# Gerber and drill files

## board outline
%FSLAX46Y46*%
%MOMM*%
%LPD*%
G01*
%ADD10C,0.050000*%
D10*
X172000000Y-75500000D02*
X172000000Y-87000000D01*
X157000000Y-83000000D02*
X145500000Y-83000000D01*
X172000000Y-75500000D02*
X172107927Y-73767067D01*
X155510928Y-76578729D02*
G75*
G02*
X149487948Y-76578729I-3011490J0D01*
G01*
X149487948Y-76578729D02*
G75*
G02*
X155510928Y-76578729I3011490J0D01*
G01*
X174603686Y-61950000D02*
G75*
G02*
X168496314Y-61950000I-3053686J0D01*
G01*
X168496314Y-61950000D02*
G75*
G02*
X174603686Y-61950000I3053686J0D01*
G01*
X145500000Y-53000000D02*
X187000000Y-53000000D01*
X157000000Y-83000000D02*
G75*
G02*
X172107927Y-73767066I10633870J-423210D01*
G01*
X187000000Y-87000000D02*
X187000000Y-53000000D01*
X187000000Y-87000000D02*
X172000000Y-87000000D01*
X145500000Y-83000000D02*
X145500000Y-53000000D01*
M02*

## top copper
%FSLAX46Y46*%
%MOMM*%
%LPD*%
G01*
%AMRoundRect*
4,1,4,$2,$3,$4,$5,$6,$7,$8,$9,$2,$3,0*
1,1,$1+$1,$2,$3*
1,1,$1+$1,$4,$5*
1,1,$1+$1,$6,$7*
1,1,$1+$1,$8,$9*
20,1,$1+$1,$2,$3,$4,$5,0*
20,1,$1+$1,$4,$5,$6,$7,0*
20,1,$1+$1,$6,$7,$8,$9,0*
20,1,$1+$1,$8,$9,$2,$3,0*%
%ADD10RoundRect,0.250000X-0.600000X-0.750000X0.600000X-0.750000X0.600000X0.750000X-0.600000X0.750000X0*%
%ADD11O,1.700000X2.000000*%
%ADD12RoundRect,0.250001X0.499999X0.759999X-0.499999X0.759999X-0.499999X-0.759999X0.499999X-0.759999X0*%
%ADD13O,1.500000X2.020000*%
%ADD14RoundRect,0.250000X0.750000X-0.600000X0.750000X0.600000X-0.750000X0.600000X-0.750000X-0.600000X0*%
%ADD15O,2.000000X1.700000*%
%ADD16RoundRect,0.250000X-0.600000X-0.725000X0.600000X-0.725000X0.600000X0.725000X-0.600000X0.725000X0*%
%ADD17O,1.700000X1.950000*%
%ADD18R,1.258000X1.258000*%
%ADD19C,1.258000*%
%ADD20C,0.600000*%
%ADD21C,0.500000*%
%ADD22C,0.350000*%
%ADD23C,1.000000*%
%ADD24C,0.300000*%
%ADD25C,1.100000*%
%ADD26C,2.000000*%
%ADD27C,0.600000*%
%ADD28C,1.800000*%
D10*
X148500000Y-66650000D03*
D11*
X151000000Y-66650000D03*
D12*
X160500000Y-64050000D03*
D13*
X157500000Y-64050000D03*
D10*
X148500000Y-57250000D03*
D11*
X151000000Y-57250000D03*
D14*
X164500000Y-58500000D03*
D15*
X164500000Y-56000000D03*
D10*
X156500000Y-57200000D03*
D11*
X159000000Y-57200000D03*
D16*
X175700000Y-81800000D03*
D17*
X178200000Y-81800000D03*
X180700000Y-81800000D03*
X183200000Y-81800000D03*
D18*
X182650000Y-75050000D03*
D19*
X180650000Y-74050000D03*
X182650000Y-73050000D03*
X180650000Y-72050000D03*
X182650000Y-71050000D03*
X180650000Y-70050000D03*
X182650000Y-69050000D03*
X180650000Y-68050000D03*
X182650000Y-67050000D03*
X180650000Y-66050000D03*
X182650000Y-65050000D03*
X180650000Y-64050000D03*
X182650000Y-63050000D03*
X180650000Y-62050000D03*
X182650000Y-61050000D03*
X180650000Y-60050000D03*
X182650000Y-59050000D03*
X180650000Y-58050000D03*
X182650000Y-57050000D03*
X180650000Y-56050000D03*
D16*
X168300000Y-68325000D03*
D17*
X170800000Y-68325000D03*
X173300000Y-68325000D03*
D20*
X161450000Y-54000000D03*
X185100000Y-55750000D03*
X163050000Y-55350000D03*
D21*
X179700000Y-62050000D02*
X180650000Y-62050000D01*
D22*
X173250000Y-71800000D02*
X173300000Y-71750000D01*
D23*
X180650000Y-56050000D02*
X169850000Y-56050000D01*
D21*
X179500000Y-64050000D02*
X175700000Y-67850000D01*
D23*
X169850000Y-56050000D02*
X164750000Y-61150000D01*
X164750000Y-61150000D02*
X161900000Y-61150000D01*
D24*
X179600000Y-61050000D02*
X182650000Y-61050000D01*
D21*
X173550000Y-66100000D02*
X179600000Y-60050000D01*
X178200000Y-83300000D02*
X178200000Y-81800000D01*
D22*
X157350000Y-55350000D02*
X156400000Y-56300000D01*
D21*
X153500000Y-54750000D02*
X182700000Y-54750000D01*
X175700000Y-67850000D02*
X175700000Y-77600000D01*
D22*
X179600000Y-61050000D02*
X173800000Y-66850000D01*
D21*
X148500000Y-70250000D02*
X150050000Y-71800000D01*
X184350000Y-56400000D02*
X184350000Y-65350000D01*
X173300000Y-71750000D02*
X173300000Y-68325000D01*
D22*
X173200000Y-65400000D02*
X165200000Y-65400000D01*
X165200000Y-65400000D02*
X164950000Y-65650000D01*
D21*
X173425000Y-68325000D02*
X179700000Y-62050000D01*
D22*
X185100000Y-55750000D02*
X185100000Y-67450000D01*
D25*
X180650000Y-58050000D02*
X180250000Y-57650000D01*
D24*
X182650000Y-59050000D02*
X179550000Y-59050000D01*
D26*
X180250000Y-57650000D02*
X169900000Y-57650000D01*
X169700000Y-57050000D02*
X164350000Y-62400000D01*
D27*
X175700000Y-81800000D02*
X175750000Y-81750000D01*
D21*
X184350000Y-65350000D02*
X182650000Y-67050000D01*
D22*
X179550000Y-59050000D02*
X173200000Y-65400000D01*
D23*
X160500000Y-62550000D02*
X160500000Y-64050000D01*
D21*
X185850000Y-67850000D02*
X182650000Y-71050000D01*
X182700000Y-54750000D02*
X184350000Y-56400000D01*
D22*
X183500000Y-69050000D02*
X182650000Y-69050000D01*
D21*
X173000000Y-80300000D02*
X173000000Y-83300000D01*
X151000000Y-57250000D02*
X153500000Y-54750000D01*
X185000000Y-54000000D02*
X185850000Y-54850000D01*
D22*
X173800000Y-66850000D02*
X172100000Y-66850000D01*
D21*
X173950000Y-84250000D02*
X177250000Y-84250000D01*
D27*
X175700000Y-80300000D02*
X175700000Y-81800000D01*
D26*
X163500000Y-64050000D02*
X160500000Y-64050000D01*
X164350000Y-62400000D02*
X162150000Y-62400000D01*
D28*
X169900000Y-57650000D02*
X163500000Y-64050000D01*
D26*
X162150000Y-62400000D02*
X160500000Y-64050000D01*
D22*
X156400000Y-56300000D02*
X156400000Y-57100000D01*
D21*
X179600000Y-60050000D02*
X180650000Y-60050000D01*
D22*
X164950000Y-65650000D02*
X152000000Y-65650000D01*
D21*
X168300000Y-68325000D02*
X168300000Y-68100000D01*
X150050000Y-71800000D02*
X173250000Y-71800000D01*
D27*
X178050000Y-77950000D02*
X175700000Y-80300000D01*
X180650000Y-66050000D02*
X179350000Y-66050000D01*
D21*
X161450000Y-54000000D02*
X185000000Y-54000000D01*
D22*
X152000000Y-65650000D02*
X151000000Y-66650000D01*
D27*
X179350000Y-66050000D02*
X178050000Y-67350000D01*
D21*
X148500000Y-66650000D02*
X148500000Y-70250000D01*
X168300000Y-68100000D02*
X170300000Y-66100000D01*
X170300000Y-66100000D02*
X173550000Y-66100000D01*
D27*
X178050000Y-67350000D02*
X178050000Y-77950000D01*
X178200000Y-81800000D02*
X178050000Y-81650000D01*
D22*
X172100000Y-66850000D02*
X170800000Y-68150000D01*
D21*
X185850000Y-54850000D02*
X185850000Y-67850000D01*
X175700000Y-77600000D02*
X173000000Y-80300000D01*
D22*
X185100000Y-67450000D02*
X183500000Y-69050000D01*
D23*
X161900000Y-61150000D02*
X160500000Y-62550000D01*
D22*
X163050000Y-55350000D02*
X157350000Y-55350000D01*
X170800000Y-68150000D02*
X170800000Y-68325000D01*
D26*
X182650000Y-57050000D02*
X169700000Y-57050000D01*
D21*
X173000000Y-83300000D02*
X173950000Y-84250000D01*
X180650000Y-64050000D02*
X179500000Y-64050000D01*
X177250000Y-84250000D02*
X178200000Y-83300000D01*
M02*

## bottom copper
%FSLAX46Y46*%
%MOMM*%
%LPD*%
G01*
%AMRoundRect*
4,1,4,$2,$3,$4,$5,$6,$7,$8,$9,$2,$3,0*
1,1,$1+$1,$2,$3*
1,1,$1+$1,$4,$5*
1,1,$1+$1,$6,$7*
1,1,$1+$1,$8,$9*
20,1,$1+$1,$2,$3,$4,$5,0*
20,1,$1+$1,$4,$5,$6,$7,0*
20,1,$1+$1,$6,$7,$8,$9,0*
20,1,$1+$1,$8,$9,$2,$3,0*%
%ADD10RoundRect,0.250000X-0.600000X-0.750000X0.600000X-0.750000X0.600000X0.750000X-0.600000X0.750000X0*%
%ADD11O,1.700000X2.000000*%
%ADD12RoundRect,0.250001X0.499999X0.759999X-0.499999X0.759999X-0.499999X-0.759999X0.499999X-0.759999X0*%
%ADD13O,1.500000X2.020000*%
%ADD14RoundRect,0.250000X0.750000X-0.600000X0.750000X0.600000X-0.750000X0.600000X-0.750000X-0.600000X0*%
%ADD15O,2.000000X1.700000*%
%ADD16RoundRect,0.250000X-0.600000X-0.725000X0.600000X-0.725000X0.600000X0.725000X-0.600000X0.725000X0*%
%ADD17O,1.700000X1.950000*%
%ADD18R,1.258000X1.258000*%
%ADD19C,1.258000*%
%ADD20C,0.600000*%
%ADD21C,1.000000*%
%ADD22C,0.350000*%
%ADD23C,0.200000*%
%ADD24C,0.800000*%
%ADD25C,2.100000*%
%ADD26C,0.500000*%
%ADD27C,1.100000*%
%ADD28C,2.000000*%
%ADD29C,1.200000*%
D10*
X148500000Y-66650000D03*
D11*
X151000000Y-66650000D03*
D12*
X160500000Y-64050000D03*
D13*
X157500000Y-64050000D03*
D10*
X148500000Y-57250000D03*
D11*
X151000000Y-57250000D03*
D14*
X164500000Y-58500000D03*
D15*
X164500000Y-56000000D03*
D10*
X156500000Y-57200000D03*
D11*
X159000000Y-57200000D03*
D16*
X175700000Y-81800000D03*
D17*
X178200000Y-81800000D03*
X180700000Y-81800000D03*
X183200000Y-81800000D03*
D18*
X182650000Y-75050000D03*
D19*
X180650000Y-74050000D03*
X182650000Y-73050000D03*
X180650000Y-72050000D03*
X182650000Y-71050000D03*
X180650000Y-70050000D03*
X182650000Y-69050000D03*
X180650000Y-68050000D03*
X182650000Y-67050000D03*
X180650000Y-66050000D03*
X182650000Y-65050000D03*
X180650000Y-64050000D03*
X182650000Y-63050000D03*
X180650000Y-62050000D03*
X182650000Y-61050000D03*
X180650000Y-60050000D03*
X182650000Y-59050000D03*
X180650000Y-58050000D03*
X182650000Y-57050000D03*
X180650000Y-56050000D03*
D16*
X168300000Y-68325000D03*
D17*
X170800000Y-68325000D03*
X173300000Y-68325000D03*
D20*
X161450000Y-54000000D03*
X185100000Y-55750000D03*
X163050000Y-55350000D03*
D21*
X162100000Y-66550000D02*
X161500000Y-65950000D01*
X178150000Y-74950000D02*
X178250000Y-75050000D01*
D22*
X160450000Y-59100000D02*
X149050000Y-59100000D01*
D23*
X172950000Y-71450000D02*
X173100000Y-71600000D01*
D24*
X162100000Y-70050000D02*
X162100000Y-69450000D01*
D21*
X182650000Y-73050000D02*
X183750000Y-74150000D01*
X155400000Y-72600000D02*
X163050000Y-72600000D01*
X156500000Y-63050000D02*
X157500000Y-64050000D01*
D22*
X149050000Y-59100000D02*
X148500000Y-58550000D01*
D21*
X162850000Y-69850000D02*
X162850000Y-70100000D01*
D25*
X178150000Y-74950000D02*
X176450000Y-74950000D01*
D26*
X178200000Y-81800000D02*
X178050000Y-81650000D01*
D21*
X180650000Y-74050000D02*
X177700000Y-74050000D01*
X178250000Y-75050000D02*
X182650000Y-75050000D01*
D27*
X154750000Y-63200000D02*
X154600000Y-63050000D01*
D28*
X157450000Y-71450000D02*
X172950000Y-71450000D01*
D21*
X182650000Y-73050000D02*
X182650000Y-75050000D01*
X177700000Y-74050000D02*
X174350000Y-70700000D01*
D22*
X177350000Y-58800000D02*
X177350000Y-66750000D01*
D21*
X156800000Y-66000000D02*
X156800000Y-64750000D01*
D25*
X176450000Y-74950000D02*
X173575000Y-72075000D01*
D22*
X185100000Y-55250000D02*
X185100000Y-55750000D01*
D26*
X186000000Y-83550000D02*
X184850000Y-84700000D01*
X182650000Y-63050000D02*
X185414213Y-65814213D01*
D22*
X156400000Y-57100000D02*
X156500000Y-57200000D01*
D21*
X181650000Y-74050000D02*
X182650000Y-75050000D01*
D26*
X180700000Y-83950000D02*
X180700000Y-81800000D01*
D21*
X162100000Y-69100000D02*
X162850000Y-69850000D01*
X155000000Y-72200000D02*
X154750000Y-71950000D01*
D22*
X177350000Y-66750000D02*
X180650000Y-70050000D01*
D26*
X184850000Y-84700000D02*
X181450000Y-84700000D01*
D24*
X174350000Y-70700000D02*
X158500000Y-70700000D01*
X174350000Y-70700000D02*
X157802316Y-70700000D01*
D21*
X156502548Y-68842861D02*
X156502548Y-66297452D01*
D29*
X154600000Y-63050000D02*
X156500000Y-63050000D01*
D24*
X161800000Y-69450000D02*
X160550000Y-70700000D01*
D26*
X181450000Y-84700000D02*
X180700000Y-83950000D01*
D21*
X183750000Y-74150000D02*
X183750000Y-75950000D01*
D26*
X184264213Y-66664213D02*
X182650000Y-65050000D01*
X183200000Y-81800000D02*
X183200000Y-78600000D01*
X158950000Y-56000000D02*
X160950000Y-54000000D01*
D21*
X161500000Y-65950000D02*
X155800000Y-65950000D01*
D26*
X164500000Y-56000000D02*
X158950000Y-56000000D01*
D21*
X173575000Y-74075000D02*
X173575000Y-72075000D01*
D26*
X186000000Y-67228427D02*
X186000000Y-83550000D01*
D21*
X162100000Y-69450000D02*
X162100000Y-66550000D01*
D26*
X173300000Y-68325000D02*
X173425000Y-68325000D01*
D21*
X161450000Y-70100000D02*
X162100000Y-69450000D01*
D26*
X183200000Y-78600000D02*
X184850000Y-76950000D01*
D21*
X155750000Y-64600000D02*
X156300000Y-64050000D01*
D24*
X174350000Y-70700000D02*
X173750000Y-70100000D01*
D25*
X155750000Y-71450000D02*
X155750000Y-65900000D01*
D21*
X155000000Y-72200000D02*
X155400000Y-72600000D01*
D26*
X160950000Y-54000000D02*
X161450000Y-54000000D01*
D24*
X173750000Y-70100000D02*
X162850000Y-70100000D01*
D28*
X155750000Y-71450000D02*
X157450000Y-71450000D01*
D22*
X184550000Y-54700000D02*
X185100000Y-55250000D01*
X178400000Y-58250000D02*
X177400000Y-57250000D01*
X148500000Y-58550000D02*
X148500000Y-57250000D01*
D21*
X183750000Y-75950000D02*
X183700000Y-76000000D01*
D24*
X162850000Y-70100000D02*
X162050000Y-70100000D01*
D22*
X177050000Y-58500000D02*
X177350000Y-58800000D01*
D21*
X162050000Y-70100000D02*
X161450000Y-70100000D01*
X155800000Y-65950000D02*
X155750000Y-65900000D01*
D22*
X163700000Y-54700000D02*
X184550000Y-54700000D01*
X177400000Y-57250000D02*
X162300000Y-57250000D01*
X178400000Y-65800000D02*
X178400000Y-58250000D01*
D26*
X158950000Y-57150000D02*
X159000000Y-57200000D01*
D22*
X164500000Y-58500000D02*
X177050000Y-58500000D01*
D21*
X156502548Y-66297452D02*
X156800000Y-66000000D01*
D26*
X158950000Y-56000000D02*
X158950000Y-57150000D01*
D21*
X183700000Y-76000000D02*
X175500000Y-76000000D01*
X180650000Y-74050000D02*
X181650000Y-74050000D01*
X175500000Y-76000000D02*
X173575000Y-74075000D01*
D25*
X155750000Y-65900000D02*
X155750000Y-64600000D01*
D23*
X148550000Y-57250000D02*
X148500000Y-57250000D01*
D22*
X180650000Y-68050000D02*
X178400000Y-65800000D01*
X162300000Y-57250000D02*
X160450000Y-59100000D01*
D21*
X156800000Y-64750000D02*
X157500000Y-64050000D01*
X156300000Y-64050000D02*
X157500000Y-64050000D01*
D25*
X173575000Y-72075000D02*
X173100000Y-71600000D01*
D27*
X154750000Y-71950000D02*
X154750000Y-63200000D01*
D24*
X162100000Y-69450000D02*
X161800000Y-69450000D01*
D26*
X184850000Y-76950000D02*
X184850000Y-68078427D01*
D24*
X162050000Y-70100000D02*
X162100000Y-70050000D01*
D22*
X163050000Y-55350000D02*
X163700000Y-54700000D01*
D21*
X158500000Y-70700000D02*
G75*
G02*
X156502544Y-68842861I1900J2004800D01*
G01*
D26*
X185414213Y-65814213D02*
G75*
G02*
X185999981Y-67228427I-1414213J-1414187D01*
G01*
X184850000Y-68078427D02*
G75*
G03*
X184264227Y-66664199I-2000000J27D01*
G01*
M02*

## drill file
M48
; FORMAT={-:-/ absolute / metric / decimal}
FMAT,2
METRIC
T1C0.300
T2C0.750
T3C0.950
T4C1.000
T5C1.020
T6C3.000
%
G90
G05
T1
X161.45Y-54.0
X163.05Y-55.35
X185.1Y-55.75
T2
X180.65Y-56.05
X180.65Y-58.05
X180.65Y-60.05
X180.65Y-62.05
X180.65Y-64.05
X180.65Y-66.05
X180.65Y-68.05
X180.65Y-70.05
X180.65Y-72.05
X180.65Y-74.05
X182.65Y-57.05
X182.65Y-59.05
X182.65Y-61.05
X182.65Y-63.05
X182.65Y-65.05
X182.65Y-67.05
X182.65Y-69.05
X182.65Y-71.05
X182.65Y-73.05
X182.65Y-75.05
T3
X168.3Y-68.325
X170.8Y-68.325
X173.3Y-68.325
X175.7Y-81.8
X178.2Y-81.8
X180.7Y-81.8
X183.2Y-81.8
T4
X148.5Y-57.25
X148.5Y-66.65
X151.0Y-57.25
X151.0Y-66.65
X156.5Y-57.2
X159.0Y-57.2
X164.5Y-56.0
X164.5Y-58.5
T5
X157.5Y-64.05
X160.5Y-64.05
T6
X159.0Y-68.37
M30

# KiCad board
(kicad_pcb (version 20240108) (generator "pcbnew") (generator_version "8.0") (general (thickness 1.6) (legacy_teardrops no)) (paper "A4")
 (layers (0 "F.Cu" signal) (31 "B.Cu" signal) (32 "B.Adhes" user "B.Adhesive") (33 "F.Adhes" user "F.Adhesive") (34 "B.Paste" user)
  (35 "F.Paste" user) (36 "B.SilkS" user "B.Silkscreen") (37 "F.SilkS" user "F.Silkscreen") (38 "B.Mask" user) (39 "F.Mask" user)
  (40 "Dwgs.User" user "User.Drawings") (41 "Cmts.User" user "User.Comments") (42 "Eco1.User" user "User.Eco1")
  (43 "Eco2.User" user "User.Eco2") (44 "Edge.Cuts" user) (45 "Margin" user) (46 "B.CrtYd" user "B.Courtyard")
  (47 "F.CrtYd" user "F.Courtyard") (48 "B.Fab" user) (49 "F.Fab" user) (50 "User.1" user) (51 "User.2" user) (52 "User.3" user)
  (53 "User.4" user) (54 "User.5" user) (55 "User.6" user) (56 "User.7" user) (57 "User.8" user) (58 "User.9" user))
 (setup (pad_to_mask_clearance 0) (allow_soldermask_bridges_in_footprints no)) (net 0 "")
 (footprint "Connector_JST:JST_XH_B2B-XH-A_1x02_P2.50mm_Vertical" (layer "F.Cu") (at 148.5 66.65)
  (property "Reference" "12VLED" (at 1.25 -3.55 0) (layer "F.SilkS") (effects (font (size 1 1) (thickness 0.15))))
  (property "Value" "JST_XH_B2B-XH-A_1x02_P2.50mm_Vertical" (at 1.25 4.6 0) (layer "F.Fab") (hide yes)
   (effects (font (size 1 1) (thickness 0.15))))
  (pad "1" thru_hole roundrect (at 0 0) (size 1.7 2) (drill 1) (layers "*.Cu" "*.Mask") (remove_unused_layers no)
   (roundrect_rratio 0.147059))
  (pad "2" thru_hole oval (at 2.5 0) (size 1.7 2) (drill 1) (layers "*.Cu" "*.Mask") (remove_unused_layers no)))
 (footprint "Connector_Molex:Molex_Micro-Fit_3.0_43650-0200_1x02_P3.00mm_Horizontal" (layer "F.Cu") (at 160.5 64.05 180)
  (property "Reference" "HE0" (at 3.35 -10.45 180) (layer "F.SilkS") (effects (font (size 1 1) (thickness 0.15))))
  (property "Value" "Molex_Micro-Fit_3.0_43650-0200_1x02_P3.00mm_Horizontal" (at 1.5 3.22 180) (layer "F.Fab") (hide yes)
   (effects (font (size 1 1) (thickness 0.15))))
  (pad "" np_thru_hole circle (at 1.5 -4.32 180) (size 3 3) (drill 3) (layers "*.Cu" "*.Mask"))
  (pad "1" thru_hole roundrect (at 0 0 180) (size 1.5 2.02) (drill 1.02) (layers "*.Cu" "*.Mask") (remove_unused_layers no)
   (roundrect_rratio 0.166667))
  (pad "2" thru_hole oval (at 3 0 180) (size 1.5 2.02) (drill 1.02) (layers "*.Cu" "*.Mask") (remove_unused_layers no)))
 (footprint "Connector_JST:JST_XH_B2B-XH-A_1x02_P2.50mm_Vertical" (layer "F.Cu") (at 148.5 57.25)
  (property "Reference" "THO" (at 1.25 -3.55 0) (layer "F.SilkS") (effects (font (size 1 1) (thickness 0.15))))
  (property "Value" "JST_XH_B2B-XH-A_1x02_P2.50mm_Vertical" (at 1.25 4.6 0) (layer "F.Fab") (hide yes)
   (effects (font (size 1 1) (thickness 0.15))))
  (pad "1" thru_hole roundrect (at 0 0) (size 1.7 2) (drill 1) (layers "*.Cu" "*.Mask") (remove_unused_layers no)
   (roundrect_rratio 0.147059))
  (pad "2" thru_hole oval (at 2.5 0) (size 1.7 2) (drill 1) (layers "*.Cu" "*.Mask") (remove_unused_layers no)))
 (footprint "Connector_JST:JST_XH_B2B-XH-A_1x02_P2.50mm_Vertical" (layer "F.Cu") (at 164.5 58.5 90)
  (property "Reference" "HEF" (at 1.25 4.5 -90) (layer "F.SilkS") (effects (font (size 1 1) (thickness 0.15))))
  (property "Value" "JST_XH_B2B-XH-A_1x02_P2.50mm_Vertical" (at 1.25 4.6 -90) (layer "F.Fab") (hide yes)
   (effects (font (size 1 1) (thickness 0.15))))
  (pad "1" thru_hole roundrect (at 0 0 90) (size 1.7 2) (drill 1) (layers "*.Cu" "*.Mask") (remove_unused_layers no)
   (roundrect_rratio 0.147059))
  (pad "2" thru_hole oval (at 2.5 0 90) (size 1.7 2) (drill 1) (layers "*.Cu" "*.Mask") (remove_unused_layers no)))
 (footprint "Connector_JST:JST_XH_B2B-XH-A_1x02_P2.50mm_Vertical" (layer "F.Cu") (at 156.5 57.2)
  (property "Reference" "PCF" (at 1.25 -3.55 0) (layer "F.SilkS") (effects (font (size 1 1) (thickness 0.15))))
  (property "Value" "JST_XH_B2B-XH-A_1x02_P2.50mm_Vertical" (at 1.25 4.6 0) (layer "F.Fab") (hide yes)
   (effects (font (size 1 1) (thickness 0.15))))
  (pad "1" thru_hole roundrect (at 0 0) (size 1.7 2) (drill 1) (layers "*.Cu" "*.Mask") (remove_unused_layers no)
   (roundrect_rratio 0.147059))
  (pad "2" thru_hole oval (at 2.5 0) (size 1.7 2) (drill 1) (layers "*.Cu" "*.Mask") (remove_unused_layers no)))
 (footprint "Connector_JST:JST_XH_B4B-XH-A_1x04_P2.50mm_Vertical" (layer "F.Cu") (at 175.7 81.8)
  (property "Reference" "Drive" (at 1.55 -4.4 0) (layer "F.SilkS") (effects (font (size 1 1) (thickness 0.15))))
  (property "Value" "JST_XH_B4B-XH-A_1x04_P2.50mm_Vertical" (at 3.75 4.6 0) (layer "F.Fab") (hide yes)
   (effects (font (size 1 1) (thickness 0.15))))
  (pad "1" thru_hole roundrect (at 0 0) (size 1.7 1.95) (drill 0.95) (layers "*.Cu" "*.Mask") (remove_unused_layers no)
   (roundrect_rratio 0.147059))
  (pad "2" thru_hole oval (at 2.5 0) (size 1.7 1.95) (drill 0.95) (layers "*.Cu" "*.Mask") (remove_unused_layers no))
  (pad "3" thru_hole oval (at 5 0) (size 1.7 1.95) (drill 0.95) (layers "*.Cu" "*.Mask") (remove_unused_layers no))
  (pad "4" thru_hole oval (at 7.5 0) (size 1.7 1.95) (drill 0.95) (layers "*.Cu" "*.Mask") (remove_unused_layers no)))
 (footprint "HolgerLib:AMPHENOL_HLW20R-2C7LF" (layer "F.Cu") (at 183.225 65.55 90)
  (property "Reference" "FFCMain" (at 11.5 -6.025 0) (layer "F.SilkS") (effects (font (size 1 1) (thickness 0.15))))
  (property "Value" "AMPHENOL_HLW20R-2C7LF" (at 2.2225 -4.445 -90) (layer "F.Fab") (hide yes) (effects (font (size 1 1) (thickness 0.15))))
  (pad "1" thru_hole rect (at -9.5 -0.575 90) (size 1.258 1.258) (drill 0.75) (layers "*.Cu" "*.Mask") (remove_unused_layers no)
   (solder_mask_margin 0.102))
  (pad "2" thru_hole circle (at -8.5 -2.575 90) (size 1.258 1.258) (drill 0.75) (layers "*.Cu" "*.Mask") (remove_unused_layers no)
   (solder_mask_margin 0.102))
  (pad "3" thru_hole circle (at -7.5 -0.575 90) (size 1.258 1.258) (drill 0.75) (layers "*.Cu" "*.Mask") (remove_unused_layers no)
   (solder_mask_margin 0.102))
  (pad "4" thru_hole circle (at -6.5 -2.575 90) (size 1.258 1.258) (drill 0.75) (layers "*.Cu" "*.Mask") (remove_unused_layers no)
   (solder_mask_margin 0.102))
  (pad "5" thru_hole circle (at -5.5 -0.575 90) (size 1.258 1.258) (drill 0.75) (layers "*.Cu" "*.Mask") (remove_unused_layers no)
   (solder_mask_margin 0.102))
  (pad "6" thru_hole circle (at -4.5 -2.575 90) (size 1.258 1.258) (drill 0.75) (layers "*.Cu" "*.Mask") (remove_unused_layers no)
   (solder_mask_margin 0.102))
  (pad "7" thru_hole circle (at -3.5 -0.575 90) (size 1.258 1.258) (drill 0.75) (layers "*.Cu" "*.Mask") (remove_unused_layers no)
   (solder_mask_margin 0.102))
  (pad "8" thru_hole circle (at -2.5 -2.575 90) (size 1.258 1.258) (drill 0.75) (layers "*.Cu" "*.Mask") (remove_unused_layers no)
   (solder_mask_margin 0.102))
  (pad "9" thru_hole circle (at -1.5 -0.575 90) (size 1.258 1.258) (drill 0.75) (layers "*.Cu" "*.Mask") (remove_unused_layers no)
   (solder_mask_margin 0.102))
  (pad "10" thru_hole circle (at -0.5 -2.575 90) (size 1.258 1.258) (drill 0.75) (layers "*.Cu" "*.Mask") (remove_unused_layers no)
   (solder_mask_margin 0.102))
  (pad "11" thru_hole circle (at 0.5 -0.575 90) (size 1.258 1.258) (drill 0.75) (layers "*.Cu" "*.Mask") (remove_unused_layers no)
   (solder_mask_margin 0.102))
  (pad "12" thru_hole circle (at 1.5 -2.575 90) (size 1.258 1.258) (drill 0.75) (layers "*.Cu" "*.Mask") (remove_unused_layers no)
   (solder_mask_margin 0.102))
  (pad "13" thru_hole circle (at 2.5 -0.575 90) (size 1.258 1.258) (drill 0.75) (layers "*.Cu" "*.Mask") (remove_unused_layers no)
   (solder_mask_margin 0.102))
  (pad "14" thru_hole circle (at 3.5 -2.575 90) (size 1.258 1.258) (drill 0.75) (layers "*.Cu" "*.Mask") (remove_unused_layers no)
   (solder_mask_margin 0.102))
  (pad "15" thru_hole circle (at 4.5 -0.575 90) (size 1.258 1.258) (drill 0.75) (layers "*.Cu" "*.Mask") (remove_unused_layers no)
   (solder_mask_margin 0.102))
  (pad "16" thru_hole circle (at 5.5 -2.575 90) (size 1.258 1.258) (drill 0.75) (layers "*.Cu" "*.Mask") (remove_unused_layers no)
   (solder_mask_margin 0.102))
  (pad "17" thru_hole circle (at 6.5 -0.575 90) (size 1.258 1.258) (drill 0.75) (layers "*.Cu" "*.Mask") (remove_unused_layers no)
   (solder_mask_margin 0.102))
  (pad "18" thru_hole circle (at 7.5 -2.575 90) (size 1.258 1.258) (drill 0.75) (layers "*.Cu" "*.Mask") (remove_unused_layers no)
   (solder_mask_margin 0.102))
  (pad "19" thru_hole circle (at 8.5 -0.575 90) (size 1.258 1.258) (drill 0.75) (layers "*.Cu" "*.Mask") (remove_unused_layers no)
   (solder_mask_margin 0.102))
  (pad "20" thru_hole circle (at 9.5 -2.575 90) (size 1.258 1.258) (drill 0.75) (layers "*.Cu" "*.Mask") (remove_unused_layers no)
   (solder_mask_margin 0.102)))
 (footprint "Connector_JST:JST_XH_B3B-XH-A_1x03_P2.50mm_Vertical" (layer "F.Cu") (at 168.3 68.325)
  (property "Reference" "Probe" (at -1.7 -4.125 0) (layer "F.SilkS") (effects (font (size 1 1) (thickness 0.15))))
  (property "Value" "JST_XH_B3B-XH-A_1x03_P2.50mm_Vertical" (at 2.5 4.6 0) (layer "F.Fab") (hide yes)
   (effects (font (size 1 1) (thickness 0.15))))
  (pad "1" thru_hole roundrect (at 0 0) (size 1.7 1.95) (drill 0.95) (layers "*.Cu" "*.Mask") (remove_unused_layers no)
   (roundrect_rratio 0.147059))
  (pad "2" thru_hole oval (at 2.5 0) (size 1.7 1.95) (drill 0.95) (layers "*.Cu" "*.Mask") (remove_unused_layers no))
  (pad "3" thru_hole oval (at 5 0) (size 1.7 1.95) (drill 0.95) (layers "*.Cu" "*.Mask") (remove_unused_layers no)))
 (gr_line (start 172 75.5) (end 172 87) (stroke (width 0.05) (type default)) (layer "Edge.Cuts"))
 (gr_line (start 157 83) (end 145.5 83) (stroke (width 0.05) (type default)) (layer "Edge.Cuts"))
 (gr_line (start 172 75.5) (end 172.107927 73.767067) (stroke (width 0.05) (type default)) (layer "Edge.Cuts"))
 (gr_circle (center 152.499438 76.578729) (end 155.510928 76.578729) (stroke (width 0.05) (type default)) (fill none) (layer "Edge.Cuts"))
 (gr_circle (center 171.55 61.95) (end 173.9 63.9) (stroke (width 0.05) (type default)) (fill none) (layer "Edge.Cuts"))
 (gr_line (start 145.5 53) (end 187 53) (stroke (width 0.05) (type default)) (layer "Edge.Cuts"))
 (gr_arc (start 157 83) (mid 162.084312 74.342422) (end 172.107927 73.767067) (stroke (width 0.05) (type default)) (layer "Edge.Cuts"))
 (gr_line (start 187 87) (end 187 53) (stroke (width 0.05) (type default)) (layer "Edge.Cuts"))
 (gr_line (start 187 87) (end 172 87) (stroke (width 0.05) (type default)) (layer "Edge.Cuts"))
 (gr_line (start 145.5 83) (end 145.5 53) (stroke (width 0.05) (type default)) (layer "Edge.Cuts"))
 (segment (start 179.7 62.05) (end 180.65 62.05) (width 0.5) (layer "F.Cu") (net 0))
 (segment (start 173.25 71.8) (end 173.3 71.75) (width 0.35) (layer "F.Cu") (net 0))
 (segment (start 180.65 56.05) (end 169.85 56.05) (width 1) (layer "F.Cu") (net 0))
 (segment (start 179.5 64.05) (end 175.7 67.85) (width 0.5) (layer "F.Cu") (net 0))
 (segment (start 169.85 56.05) (end 164.75 61.15) (width 1) (layer "F.Cu") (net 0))
 (segment (start 164.75 61.15) (end 161.9 61.15) (width 1) (layer "F.Cu") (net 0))
 (segment (start 179.6 61.05) (end 182.65 61.05) (width 0.3) (layer "F.Cu") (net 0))
 (segment (start 173.55 66.1) (end 179.6 60.05) (width 0.5) (layer "F.Cu") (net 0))
 (segment (start 178.2 83.3) (end 178.2 81.8) (width 0.5) (layer "F.Cu") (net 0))
 (segment (start 157.35 55.35) (end 156.4 56.3) (width 0.35) (layer "F.Cu") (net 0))
 (segment (start 153.5 54.75) (end 182.7 54.75) (width 0.5) (layer "F.Cu") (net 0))
 (segment (start 175.7 67.85) (end 175.7 77.6) (width 0.5) (layer "F.Cu") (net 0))
 (segment (start 179.6 61.05) (end 173.8 66.85) (width 0.35) (layer "F.Cu") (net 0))
 (segment (start 148.5 70.25) (end 150.05 71.8) (width 0.5) (layer "F.Cu") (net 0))
 (segment (start 184.35 56.4) (end 184.35 65.35) (width 0.5) (layer "F.Cu") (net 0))
 (segment (start 173.3 71.75) (end 173.3 68.325) (width 0.5) (layer "F.Cu") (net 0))
 (segment (start 173.2 65.4) (end 165.2 65.4) (width 0.35) (layer "F.Cu") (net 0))
 (segment (start 165.2 65.4) (end 164.95 65.65) (width 0.35) (layer "F.Cu") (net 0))
 (segment (start 173.425 68.325) (end 179.7 62.05) (width 0.5) (layer "F.Cu") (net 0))
 (segment (start 185.1 55.75) (end 185.1 67.45) (width 0.35) (layer "F.Cu") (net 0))
 (segment (start 180.65 58.05) (end 180.25 57.65) (width 1.1) (layer "F.Cu") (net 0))
 (segment (start 182.65 59.05) (end 179.55 59.05) (width 0.3) (layer "F.Cu") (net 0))
 (segment (start 180.25 57.65) (end 169.9 57.65) (width 2) (layer "F.Cu") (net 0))
 (segment (start 169.7 57.05) (end 164.35 62.4) (width 2) (layer "F.Cu") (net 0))
 (segment (start 175.7 81.8) (end 175.75 81.75) (width 0.6) (layer "F.Cu") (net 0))
 (segment (start 184.35 65.35) (end 182.65 67.05) (width 0.5) (layer "F.Cu") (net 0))
 (segment (start 179.55 59.05) (end 173.2 65.4) (width 0.35) (layer "F.Cu") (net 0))
 (segment (start 160.5 62.55) (end 160.5 64.05) (width 1) (layer "F.Cu") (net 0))
 (segment (start 185.85 67.85) (end 182.65 71.05) (width 0.5) (layer "F.Cu") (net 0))
 (segment (start 182.7 54.75) (end 184.35 56.4) (width 0.5) (layer "F.Cu") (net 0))
 (segment (start 183.5 69.05) (end 182.65 69.05) (width 0.35) (layer "F.Cu") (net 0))
 (segment (start 173 80.3) (end 173 83.3) (width 0.5) (layer "F.Cu") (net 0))
 (segment (start 151 57.25) (end 153.5 54.75) (width 0.5) (layer "F.Cu") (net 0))
 (segment (start 185 54) (end 185.85 54.85) (width 0.5) (layer "F.Cu") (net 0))
 (segment (start 173.8 66.85) (end 172.1 66.85) (width 0.35) (layer "F.Cu") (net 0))
 (segment (start 173.95 84.25) (end 177.25 84.25) (width 0.5) (layer "F.Cu") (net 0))
 (segment (start 175.7 80.3) (end 175.7 81.8) (width 0.6) (layer "F.Cu") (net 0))
 (segment (start 163.5 64.05) (end 160.5 64.05) (width 2) (layer "F.Cu") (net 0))
 (segment (start 164.35 62.4) (end 162.15 62.4) (width 2) (layer "F.Cu") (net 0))
 (segment (start 169.9 57.65) (end 163.5 64.05) (width 1.8) (layer "F.Cu") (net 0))
 (segment (start 162.15 62.4) (end 160.5 64.05) (width 2) (layer "F.Cu") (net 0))
 (segment (start 156.4 56.3) (end 156.4 57.1) (width 0.35) (layer "F.Cu") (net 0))
 (segment (start 179.6 60.05) (end 180.65 60.05) (width 0.5) (layer "F.Cu") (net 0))
 (segment (start 164.95 65.65) (end 152 65.65) (width 0.35) (layer "F.Cu") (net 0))
 (segment (start 168.3 68.325) (end 168.3 68.1) (width 0.5) (layer "F.Cu") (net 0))
 (segment (start 150.05 71.8) (end 173.25 71.8) (width 0.5) (layer "F.Cu") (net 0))
 (segment (start 178.05 77.95) (end 175.7 80.3) (width 0.6) (layer "F.Cu") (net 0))
 (segment (start 180.65 66.05) (end 179.35 66.05) (width 0.6) (layer "F.Cu") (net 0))
 (segment (start 161.45 54) (end 185 54) (width 0.5) (layer "F.Cu") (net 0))
 (segment (start 152 65.65) (end 151 66.65) (width 0.35) (layer "F.Cu") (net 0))
 (segment (start 179.35 66.05) (end 178.05 67.35) (width 0.6) (layer "F.Cu") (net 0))
 (segment (start 148.5 66.65) (end 148.5 70.25) (width 0.5) (layer "F.Cu") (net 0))
 (segment (start 168.3 68.1) (end 170.3 66.1) (width 0.5) (layer "F.Cu") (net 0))
 (segment (start 170.3 66.1) (end 173.55 66.1) (width 0.5) (layer "F.Cu") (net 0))
 (segment (start 178.05 67.35) (end 178.05 77.95) (width 0.6) (layer "F.Cu") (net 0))
 (segment (start 178.2 81.8) (end 178.05 81.65) (width 0.6) (layer "F.Cu") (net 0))
 (segment (start 172.1 66.85) (end 170.8 68.15) (width 0.35) (layer "F.Cu") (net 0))
 (segment (start 185.85 54.85) (end 185.85 67.85) (width 0.5) (layer "F.Cu") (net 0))
 (segment (start 175.7 77.6) (end 173 80.3) (width 0.5) (layer "F.Cu") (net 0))
 (segment (start 185.1 67.45) (end 183.5 69.05) (width 0.35) (layer "F.Cu") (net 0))
 (segment (start 161.9 61.15) (end 160.5 62.55) (width 1) (layer "F.Cu") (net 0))
 (segment (start 163.05 55.35) (end 157.35 55.35) (width 0.35) (layer "F.Cu") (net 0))
 (segment (start 170.8 68.15) (end 170.8 68.325) (width 0.35) (layer "F.Cu") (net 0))
 (segment (start 182.65 57.05) (end 169.7 57.05) (width 2) (layer "F.Cu") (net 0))
 (segment (start 173 83.3) (end 173.95 84.25) (width 0.5) (layer "F.Cu") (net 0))
 (segment (start 180.65 64.05) (end 179.5 64.05) (width 0.5) (layer "F.Cu") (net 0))
 (segment (start 177.25 84.25) (end 178.2 83.3) (width 0.5) (layer "F.Cu") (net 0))
 (via (at 161.45 54) (size 0.6) (drill 0.3) (layers "F.Cu" "B.Cu") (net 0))
 (via (at 185.1 55.75) (size 0.6) (drill 0.3) (layers "F.Cu" "B.Cu") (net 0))
 (via (at 163.05 55.35) (size 0.6) (drill 0.3) (layers "F.Cu" "B.Cu") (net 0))
 (segment (start 162.1 66.55) (end 161.5 65.95) (width 1) (layer "B.Cu") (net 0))
 (segment (start 178.15 74.95) (end 178.25 75.05) (width 1) (layer "B.Cu") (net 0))
 (segment (start 160.45 59.1) (end 149.05 59.1) (width 0.35) (layer "B.Cu") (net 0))
 (segment (start 172.95 71.45) (end 173.1 71.6) (width 0.2) (layer "B.Cu") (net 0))
 (segment (start 162.1 70.05) (end 162.1 69.45) (width 0.8) (layer "B.Cu") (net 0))
 (segment (start 182.65 73.05) (end 183.75 74.15) (width 1) (layer "B.Cu") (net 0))
 (segment (start 155.4 72.6) (end 163.05 72.6) (width 1) (layer "B.Cu") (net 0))
 (segment (start 156.5 63.05) (end 157.5 64.05) (width 1) (layer "B.Cu") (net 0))
 (segment (start 149.05 59.1) (end 148.5 58.55) (width 0.35) (layer "B.Cu") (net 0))
 (segment (start 162.85 69.85) (end 162.85 70.1) (width 1) (layer "B.Cu") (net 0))
 (segment (start 178.15 74.95) (end 176.45 74.95) (width 2.1) (layer "B.Cu") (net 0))
 (segment (start 178.2 81.8) (end 178.05 81.65) (width 0.5) (layer "B.Cu") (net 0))
 (segment (start 180.65 74.05) (end 177.7 74.05) (width 1) (layer "B.Cu") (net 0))
 (segment (start 178.25 75.05) (end 182.65 75.05) (width 1) (layer "B.Cu") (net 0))
 (segment (start 154.75 63.2) (end 154.6 63.05) (width 1.1) (layer "B.Cu") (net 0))
 (segment (start 157.45 71.45) (end 172.95 71.45) (width 2) (layer "B.Cu") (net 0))
 (segment (start 182.65 73.05) (end 182.65 75.05) (width 1) (layer "B.Cu") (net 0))
 (segment (start 177.7 74.05) (end 174.35 70.7) (width 1) (layer "B.Cu") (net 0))
 (segment (start 177.35 58.8) (end 177.35 66.75) (width 0.35) (layer "B.Cu") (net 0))
 (segment (start 156.8 66) (end 156.8 64.75) (width 1) (layer "B.Cu") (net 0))
 (segment (start 176.45 74.95) (end 173.575 72.075) (width 2.1) (layer "B.Cu") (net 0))
 (segment (start 185.1 55.25) (end 185.1 55.75) (width 0.35) (layer "B.Cu") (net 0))
 (segment (start 186 83.55) (end 184.85 84.7) (width 0.5) (layer "B.Cu") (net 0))
 (segment (start 182.65 63.05) (end 185.414213 65.814213) (width 0.5) (layer "B.Cu") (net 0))
 (segment (start 156.4 57.1) (end 156.5 57.2) (width 0.35) (layer "B.Cu") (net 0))
 (segment (start 181.65 74.05) (end 182.65 75.05) (width 1) (layer "B.Cu") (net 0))
 (segment (start 180.7 83.95) (end 180.7 81.8) (width 0.5) (layer "B.Cu") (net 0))
 (segment (start 162.1 69.1) (end 162.85 69.85) (width 1) (layer "B.Cu") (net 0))
 (segment (start 155 72.2) (end 154.75 71.95) (width 1) (layer "B.Cu") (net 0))
 (segment (start 177.35 66.75) (end 180.65 70.05) (width 0.35) (layer "B.Cu") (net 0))
 (segment (start 184.85 84.7) (end 181.45 84.7) (width 0.5) (layer "B.Cu") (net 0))
 (segment (start 174.35 70.7) (end 158.5 70.7) (width 0.8) (layer "B.Cu") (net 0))
 (segment (start 174.35 70.7) (end 157.802316 70.7) (width 0.8) (layer "B.Cu") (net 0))
 (segment (start 156.502548 68.842861) (end 156.502548 66.297452) (width 1) (layer "B.Cu") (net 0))
 (segment (start 154.6 63.05) (end 156.5 63.05) (width 1.2) (layer "B.Cu") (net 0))
 (segment (start 161.8 69.45) (end 160.55 70.7) (width 0.8) (layer "B.Cu") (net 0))
 (segment (start 181.45 84.7) (end 180.7 83.95) (width 0.5) (layer "B.Cu") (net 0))
 (segment (start 183.75 74.15) (end 183.75 75.95) (width 1) (layer "B.Cu") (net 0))
 (segment (start 184.264213 66.664213) (end 182.65 65.05) (width 0.5) (layer "B.Cu") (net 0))
 (segment (start 183.2 81.8) (end 183.2 78.6) (width 0.5) (layer "B.Cu") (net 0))
 (segment (start 158.95 56) (end 160.95 54) (width 0.5) (layer "B.Cu") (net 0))
 (segment (start 161.5 65.95) (end 155.8 65.95) (width 1) (layer "B.Cu") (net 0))
 (segment (start 164.5 56) (end 158.95 56) (width 0.5) (layer "B.Cu") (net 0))
 (segment (start 173.575 74.075) (end 173.575 72.075) (width 1) (layer "B.Cu") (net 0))
 (segment (start 186 67.228427) (end 186 83.55) (width 0.5) (layer "B.Cu") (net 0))
 (segment (start 162.1 69.45) (end 162.1 66.55) (width 1) (layer "B.Cu") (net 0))
 (segment (start 173.3 68.325) (end 173.425 68.325) (width 0.5) (layer "B.Cu") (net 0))
 (segment (start 161.45 70.1) (end 162.1 69.45) (width 1) (layer "B.Cu") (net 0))
 (segment (start 183.2 78.6) (end 184.85 76.95) (width 0.5) (layer "B.Cu") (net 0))
 (segment (start 155.75 64.6) (end 156.3 64.05) (width 1) (layer "B.Cu") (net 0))
 (segment (start 174.35 70.7) (end 173.75 70.1) (width 0.8) (layer "B.Cu") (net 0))
 (segment (start 155.75 71.45) (end 155.75 65.9) (width 2.1) (layer "B.Cu") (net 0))
 (segment (start 155 72.2) (end 155.4 72.6) (width 1) (layer "B.Cu") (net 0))
 (segment (start 160.95 54) (end 161.45 54) (width 0.5) (layer "B.Cu") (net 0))
 (segment (start 173.75 70.1) (end 162.85 70.1) (width 0.8) (layer "B.Cu") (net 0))
 (segment (start 155.75 71.45) (end 157.45 71.45) (width 2) (layer "B.Cu") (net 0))
 (segment (start 184.55 54.7) (end 185.1 55.25) (width 0.35) (layer "B.Cu") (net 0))
 (segment (start 178.4 58.25) (end 177.4 57.25) (width 0.35) (layer "B.Cu") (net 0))
 (segment (start 148.5 58.55) (end 148.5 57.25) (width 0.35) (layer "B.Cu") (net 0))
 (segment (start 183.75 75.95) (end 183.7 76) (width 1) (layer "B.Cu") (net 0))
 (segment (start 162.85 70.1) (end 162.05 70.1) (width 0.8) (layer "B.Cu") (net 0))
 (segment (start 177.05 58.5) (end 177.35 58.8) (width 0.35) (layer "B.Cu") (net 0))
 (segment (start 162.05 70.1) (end 161.45 70.1) (width 1) (layer "B.Cu") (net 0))
 (segment (start 155.8 65.95) (end 155.75 65.9) (width 1) (layer "B.Cu") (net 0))
 (segment (start 163.7 54.7) (end 184.55 54.7) (width 0.35) (layer "B.Cu") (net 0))
 (segment (start 177.4 57.25) (end 162.3 57.25) (width 0.35) (layer "B.Cu") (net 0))
 (segment (start 178.4 65.8) (end 178.4 58.25) (width 0.35) (layer "B.Cu") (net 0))
 (segment (start 158.95 57.15) (end 159 57.2) (width 0.5) (layer "B.Cu") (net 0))
 (segment (start 164.5 58.5) (end 177.05 58.5) (width 0.35) (layer "B.Cu") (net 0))
 (segment (start 156.502548 66.297452) (end 156.8 66) (width 1) (layer "B.Cu") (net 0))
 (segment (start 158.95 56) (end 158.95 57.15) (width 0.5) (layer "B.Cu") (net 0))
 (segment (start 183.7 76) (end 175.5 76) (width 1) (layer "B.Cu") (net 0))
 (segment (start 180.65 74.05) (end 181.65 74.05) (width 1) (layer "B.Cu") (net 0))
 (segment (start 175.5 76) (end 173.575 74.075) (width 1) (layer "B.Cu") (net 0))
 (segment (start 155.75 65.9) (end 155.75 64.6) (width 2.1) (layer "B.Cu") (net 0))
 (segment (start 148.55 57.25) (end 148.5 57.25) (width 0.2) (layer "B.Cu") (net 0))
 (segment (start 180.65 68.05) (end 178.4 65.8) (width 0.35) (layer "B.Cu") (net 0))
 (segment (start 162.3 57.25) (end 160.45 59.1) (width 0.35) (layer "B.Cu") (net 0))
 (segment (start 156.8 64.75) (end 157.5 64.05) (width 1) (layer "B.Cu") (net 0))
 (segment (start 156.3 64.05) (end 157.5 64.05) (width 1) (layer "B.Cu") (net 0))
 (segment (start 173.575 72.075) (end 173.1 71.6) (width 2.1) (layer "B.Cu") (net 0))
 (segment (start 154.75 71.95) (end 154.75 63.2) (width 1.1) (layer "B.Cu") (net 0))
 (segment (start 162.1 69.45) (end 161.8 69.45) (width 0.8) (layer "B.Cu") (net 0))
 (segment (start 184.85 76.95) (end 184.85 68.078427) (width 0.5) (layer "B.Cu") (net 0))
 (segment (start 162.05 70.1) (end 162.1 70.05) (width 0.8) (layer "B.Cu") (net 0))
 (segment (start 163.05 55.35) (end 163.7 54.7) (width 0.35) (layer "B.Cu") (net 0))
 (arc (start 158.5 70.7) (mid 157.137164 70.163789) (end 156.502548 68.842861) (width 1) (layer "B.Cu") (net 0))
 (arc (start 185.414213 65.814213) (mid 185.847759 66.46306) (end 186 67.228427) (width 0.5) (layer "B.Cu") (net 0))
 (arc (start 184.85 68.078427) (mid 184.697759 67.31306) (end 184.264213 66.664213) (width 0.5) (layer "B.Cu") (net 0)))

